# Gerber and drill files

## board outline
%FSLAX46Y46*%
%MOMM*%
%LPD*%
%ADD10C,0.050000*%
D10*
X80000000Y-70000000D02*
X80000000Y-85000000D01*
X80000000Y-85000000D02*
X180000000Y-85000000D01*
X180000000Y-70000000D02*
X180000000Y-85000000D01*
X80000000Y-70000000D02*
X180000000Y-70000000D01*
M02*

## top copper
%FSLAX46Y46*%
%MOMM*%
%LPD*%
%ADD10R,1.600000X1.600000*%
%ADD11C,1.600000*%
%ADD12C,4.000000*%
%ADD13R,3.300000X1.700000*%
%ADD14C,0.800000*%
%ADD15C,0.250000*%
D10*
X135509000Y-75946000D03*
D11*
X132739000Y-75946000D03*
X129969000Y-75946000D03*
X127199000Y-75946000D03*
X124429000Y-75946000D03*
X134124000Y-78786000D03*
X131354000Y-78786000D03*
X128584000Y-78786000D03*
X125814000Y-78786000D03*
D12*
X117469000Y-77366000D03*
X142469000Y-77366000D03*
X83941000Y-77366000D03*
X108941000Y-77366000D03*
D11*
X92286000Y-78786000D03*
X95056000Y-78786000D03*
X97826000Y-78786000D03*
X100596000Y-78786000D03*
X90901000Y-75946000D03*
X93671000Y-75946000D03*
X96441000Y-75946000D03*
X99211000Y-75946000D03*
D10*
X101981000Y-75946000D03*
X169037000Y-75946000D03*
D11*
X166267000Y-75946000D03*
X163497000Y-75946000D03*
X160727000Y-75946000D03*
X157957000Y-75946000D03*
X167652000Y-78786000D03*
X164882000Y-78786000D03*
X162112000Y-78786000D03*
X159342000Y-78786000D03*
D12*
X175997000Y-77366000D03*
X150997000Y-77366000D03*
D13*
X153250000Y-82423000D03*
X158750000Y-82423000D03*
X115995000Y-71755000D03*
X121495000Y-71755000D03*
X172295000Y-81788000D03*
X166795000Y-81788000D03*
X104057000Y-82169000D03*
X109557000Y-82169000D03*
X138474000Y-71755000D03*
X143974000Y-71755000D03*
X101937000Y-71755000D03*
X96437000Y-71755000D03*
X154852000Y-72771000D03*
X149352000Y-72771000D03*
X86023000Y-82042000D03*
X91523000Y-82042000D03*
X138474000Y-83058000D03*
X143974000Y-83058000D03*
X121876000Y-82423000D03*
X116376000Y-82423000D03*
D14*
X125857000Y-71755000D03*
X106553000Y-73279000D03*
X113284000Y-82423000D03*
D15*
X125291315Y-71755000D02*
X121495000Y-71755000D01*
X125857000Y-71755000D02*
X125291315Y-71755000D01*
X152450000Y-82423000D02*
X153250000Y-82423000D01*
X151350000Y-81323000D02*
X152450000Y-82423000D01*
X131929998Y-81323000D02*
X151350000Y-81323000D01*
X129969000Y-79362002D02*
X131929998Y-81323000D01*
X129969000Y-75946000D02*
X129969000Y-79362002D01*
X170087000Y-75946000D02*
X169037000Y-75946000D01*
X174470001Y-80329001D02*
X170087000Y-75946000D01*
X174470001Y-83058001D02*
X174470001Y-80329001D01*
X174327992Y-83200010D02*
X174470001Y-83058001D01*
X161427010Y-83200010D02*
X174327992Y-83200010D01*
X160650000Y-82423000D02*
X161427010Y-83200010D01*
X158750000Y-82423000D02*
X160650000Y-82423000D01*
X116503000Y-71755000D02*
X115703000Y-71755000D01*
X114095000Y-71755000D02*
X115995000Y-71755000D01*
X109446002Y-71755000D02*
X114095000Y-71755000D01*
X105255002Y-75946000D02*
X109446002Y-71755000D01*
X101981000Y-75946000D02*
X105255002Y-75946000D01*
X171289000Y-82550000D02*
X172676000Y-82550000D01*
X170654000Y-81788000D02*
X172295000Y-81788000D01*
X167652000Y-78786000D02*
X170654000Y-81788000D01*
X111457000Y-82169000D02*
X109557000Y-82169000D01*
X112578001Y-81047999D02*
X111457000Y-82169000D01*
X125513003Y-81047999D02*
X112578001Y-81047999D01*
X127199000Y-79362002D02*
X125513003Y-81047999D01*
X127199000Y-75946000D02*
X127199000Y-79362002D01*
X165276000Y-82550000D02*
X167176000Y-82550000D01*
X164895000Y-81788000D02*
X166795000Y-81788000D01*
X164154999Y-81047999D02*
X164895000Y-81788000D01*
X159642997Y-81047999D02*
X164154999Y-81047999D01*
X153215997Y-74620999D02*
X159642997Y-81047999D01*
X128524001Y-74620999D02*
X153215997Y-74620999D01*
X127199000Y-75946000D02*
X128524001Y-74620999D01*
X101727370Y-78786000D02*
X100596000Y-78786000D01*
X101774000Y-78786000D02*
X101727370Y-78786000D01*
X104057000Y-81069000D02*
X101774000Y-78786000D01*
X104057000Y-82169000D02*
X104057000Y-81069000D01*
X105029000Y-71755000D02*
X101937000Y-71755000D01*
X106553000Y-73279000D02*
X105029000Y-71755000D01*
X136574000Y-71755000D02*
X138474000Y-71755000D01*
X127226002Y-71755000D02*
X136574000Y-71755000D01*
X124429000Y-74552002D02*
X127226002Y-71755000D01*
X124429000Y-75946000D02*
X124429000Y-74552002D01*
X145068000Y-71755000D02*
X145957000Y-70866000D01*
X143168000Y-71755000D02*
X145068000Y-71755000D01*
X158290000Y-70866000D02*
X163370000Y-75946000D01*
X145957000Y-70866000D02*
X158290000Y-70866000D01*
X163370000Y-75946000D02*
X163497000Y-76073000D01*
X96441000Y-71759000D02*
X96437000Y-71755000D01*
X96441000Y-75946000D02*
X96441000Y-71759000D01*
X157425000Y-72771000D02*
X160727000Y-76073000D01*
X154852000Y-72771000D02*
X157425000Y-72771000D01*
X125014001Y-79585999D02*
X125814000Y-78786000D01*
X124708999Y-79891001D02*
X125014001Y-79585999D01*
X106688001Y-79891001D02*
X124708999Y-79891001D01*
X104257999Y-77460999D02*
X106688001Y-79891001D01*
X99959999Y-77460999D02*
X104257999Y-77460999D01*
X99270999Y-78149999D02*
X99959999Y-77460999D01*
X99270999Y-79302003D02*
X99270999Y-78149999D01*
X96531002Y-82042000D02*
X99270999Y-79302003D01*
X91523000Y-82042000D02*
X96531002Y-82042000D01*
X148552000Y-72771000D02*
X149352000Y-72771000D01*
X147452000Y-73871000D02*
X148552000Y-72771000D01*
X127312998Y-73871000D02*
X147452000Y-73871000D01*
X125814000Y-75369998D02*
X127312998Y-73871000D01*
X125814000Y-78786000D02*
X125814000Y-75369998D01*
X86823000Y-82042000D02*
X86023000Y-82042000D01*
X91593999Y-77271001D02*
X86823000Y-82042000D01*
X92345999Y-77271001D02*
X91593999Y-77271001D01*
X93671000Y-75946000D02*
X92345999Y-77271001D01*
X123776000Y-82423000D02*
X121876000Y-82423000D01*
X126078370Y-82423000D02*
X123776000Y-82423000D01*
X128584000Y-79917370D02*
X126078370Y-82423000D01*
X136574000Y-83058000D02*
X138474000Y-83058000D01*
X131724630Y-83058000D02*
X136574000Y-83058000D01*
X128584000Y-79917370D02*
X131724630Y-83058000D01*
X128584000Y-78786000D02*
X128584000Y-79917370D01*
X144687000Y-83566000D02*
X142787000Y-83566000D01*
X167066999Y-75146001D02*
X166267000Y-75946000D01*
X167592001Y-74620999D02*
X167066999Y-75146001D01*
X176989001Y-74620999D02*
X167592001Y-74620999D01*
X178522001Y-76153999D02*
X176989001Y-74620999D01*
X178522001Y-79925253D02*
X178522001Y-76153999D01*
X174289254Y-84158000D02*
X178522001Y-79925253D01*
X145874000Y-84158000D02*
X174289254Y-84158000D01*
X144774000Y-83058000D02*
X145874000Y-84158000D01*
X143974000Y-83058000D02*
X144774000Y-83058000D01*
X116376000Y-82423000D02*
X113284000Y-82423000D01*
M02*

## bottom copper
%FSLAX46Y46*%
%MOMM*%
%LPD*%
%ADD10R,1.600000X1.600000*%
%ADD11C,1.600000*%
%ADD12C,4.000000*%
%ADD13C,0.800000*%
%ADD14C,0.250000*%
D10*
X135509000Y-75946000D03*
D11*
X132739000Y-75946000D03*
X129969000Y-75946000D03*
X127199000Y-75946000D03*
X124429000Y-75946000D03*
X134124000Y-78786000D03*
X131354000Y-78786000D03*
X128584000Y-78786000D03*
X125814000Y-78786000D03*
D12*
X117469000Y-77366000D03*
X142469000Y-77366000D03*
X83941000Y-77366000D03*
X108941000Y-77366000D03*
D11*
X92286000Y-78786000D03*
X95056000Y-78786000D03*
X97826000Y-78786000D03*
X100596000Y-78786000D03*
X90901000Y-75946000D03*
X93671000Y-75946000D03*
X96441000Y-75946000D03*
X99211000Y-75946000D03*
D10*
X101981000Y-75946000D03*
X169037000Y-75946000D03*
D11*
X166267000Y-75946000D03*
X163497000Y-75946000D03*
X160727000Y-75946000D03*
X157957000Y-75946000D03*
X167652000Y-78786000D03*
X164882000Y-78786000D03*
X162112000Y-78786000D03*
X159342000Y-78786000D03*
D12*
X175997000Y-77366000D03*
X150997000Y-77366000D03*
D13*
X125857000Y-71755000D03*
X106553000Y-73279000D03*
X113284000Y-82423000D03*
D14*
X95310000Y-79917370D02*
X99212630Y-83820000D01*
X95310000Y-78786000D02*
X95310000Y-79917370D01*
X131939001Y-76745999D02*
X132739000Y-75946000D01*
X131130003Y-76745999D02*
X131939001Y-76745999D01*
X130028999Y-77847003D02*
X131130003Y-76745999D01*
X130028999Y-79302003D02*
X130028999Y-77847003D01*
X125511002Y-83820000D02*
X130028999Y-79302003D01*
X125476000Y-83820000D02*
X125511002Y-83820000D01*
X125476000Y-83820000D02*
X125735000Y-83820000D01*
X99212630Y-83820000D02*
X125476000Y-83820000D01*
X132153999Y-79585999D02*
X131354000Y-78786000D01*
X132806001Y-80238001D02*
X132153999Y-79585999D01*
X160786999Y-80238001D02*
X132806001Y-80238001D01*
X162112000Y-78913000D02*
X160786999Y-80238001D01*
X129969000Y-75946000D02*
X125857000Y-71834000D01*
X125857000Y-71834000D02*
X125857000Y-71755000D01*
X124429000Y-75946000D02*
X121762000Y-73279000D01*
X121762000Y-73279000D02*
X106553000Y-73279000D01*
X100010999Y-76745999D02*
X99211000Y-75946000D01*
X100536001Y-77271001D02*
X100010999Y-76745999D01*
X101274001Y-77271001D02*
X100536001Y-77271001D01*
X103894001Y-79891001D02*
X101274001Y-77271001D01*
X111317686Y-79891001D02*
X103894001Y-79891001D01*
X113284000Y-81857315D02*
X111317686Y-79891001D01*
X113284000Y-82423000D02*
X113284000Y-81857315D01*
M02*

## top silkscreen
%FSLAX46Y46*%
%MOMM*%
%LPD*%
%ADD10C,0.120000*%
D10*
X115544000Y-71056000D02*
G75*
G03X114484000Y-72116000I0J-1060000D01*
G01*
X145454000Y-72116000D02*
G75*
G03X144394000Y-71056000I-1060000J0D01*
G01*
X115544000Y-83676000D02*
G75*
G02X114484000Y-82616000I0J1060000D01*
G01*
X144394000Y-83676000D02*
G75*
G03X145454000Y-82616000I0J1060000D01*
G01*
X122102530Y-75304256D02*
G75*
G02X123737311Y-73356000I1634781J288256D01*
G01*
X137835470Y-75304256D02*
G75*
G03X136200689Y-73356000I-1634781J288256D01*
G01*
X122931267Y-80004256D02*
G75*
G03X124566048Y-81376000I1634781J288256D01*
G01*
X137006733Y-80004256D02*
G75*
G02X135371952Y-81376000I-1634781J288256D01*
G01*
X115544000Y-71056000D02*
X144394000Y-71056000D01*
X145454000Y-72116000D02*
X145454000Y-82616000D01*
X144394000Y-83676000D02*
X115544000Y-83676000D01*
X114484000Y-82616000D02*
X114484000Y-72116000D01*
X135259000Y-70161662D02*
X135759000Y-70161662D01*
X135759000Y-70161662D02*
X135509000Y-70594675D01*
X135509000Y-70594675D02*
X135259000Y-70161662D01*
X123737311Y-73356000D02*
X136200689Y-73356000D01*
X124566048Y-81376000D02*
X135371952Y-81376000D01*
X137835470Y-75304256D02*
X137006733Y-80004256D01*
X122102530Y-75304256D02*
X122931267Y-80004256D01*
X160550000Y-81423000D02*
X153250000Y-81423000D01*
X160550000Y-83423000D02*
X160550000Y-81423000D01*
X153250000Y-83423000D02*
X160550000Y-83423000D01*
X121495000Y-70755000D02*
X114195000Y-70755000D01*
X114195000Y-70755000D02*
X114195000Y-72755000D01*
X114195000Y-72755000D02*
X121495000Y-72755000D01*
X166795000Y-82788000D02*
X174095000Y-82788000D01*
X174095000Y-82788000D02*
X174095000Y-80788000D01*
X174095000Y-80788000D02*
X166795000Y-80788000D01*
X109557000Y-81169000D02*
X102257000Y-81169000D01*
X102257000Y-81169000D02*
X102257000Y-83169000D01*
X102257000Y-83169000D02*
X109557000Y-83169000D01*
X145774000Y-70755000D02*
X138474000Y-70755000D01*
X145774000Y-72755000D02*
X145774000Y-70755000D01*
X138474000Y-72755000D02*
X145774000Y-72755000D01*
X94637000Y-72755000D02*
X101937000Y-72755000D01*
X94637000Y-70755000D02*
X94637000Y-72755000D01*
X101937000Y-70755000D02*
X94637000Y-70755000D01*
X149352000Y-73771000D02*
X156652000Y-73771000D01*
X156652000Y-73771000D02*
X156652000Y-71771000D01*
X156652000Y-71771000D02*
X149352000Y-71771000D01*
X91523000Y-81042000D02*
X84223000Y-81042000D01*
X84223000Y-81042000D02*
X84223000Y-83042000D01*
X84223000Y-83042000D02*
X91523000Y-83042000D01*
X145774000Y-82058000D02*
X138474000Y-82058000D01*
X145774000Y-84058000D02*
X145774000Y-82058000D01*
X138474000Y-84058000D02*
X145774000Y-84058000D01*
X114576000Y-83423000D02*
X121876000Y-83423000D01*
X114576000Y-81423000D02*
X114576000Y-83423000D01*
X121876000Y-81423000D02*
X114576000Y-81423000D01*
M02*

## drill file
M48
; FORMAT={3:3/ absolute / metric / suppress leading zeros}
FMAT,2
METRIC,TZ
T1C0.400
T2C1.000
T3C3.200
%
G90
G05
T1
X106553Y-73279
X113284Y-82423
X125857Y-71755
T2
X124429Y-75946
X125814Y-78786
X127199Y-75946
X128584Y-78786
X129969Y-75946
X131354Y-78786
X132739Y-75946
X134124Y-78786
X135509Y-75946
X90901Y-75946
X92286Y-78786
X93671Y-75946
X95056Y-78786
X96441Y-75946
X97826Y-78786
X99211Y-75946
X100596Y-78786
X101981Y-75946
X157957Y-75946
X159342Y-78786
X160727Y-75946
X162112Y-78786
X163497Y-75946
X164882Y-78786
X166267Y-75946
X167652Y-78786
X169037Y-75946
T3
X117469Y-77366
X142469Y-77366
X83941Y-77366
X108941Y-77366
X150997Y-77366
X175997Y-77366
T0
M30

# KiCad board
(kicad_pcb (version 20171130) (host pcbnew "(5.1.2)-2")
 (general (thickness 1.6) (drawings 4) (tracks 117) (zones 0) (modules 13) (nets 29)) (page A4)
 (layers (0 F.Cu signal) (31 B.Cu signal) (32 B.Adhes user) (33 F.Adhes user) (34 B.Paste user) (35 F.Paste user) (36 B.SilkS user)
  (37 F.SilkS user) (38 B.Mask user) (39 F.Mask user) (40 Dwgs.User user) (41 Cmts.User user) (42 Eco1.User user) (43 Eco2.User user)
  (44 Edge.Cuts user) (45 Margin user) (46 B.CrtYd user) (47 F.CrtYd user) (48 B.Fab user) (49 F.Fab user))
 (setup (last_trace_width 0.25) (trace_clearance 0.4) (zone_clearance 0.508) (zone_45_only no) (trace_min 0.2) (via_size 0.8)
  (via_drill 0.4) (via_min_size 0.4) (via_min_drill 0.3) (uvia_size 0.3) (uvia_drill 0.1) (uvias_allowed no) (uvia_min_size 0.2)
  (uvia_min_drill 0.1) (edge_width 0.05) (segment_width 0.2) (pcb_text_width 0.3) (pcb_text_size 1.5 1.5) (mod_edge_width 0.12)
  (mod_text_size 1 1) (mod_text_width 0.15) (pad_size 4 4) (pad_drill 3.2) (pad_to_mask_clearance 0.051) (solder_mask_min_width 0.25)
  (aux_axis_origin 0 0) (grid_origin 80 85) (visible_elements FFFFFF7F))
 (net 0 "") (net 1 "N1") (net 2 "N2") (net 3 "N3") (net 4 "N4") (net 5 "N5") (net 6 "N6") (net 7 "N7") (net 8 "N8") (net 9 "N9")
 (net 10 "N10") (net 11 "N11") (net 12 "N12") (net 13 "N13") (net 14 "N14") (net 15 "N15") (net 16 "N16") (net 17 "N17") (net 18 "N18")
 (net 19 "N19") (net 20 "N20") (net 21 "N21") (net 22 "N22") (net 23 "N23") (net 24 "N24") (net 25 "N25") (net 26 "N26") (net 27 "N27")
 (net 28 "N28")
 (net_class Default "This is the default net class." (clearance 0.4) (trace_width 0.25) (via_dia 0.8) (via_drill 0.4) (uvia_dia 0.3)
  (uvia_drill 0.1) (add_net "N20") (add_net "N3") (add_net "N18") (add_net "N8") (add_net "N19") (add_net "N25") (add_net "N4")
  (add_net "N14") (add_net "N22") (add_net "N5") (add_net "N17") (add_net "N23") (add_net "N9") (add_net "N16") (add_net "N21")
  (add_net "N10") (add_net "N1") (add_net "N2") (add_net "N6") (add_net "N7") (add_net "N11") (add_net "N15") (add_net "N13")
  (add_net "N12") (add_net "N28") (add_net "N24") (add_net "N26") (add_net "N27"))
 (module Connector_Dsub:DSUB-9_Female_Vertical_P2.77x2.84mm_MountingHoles (layer F.Cu) (at 135.509 75.946)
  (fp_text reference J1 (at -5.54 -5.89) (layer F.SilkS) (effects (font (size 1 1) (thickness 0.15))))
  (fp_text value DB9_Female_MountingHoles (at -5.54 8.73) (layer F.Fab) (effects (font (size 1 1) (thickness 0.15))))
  (fp_arc (start -19.965 -3.83) (end -21.025 -3.83) (angle 90) (layer F.SilkS) (width 0.12))
  (fp_arc (start 8.885 -3.83) (end 8.885 -4.89) (angle 90) (layer F.SilkS) (width 0.12))
  (fp_arc (start -19.965 6.67) (end -21.025 6.67) (angle -90) (layer F.SilkS) (width 0.12))
  (fp_arc (start 8.885 6.67) (end 9.945 6.67) (angle 90) (layer F.SilkS) (width 0.12))
  (fp_arc (start -11.771689 -0.93) (end -11.771689 -2.59) (angle -100) (layer F.SilkS) (width 0.12))
  (fp_arc (start 0.691689 -0.93) (end 0.691689 -2.59) (angle 100) (layer F.SilkS) (width 0.12))
  (fp_arc (start -10.942952 3.77) (end -10.942952 5.43) (angle 80) (layer F.SilkS) (width 0.12))
  (fp_arc (start -0.137048 3.77) (end -0.137048 5.43) (angle -80) (layer F.SilkS) (width 0.12))
  (fp_line (start -19.965 -4.89) (end 8.885 -4.89) (layer F.SilkS) (width 0.12))
  (fp_line (start 9.945 -3.83) (end 9.945 6.67) (layer F.SilkS) (width 0.12))
  (fp_line (start 8.885 7.73) (end -19.965 7.73) (layer F.SilkS) (width 0.12))
  (fp_line (start -21.025 6.67) (end -21.025 -3.83) (layer F.SilkS) (width 0.12))
  (fp_line (start -0.25 -5.784338) (end 0.25 -5.784338) (layer F.SilkS) (width 0.12))
  (fp_line (start 0.25 -5.784338) (end 0 -5.351325) (layer F.SilkS) (width 0.12))
  (fp_line (start 0 -5.351325) (end -0.25 -5.784338) (layer F.SilkS) (width 0.12))
  (fp_line (start -11.771689 -2.59) (end 0.691689 -2.59) (layer F.SilkS) (width 0.12))
  (fp_line (start -10.942952 5.43) (end -0.137048 5.43) (layer F.SilkS) (width 0.12))
  (fp_line (start 2.32647 -0.641744) (end 1.497733 4.058256) (layer F.SilkS) (width 0.12))
  (fp_line (start -13.40647 -0.641744) (end -12.577733 4.058256) (layer F.SilkS) (width 0.12))
  (pad 1 thru_hole rect (at 0 0) (size 1.6 1.6) (drill 1) (layers *.Cu *.Mask) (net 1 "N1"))
  (pad 2 thru_hole circle (at -2.77 0) (size 1.6 1.6) (drill 1) (layers *.Cu *.Mask) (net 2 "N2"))
  (pad 3 thru_hole circle (at -5.54 0) (size 1.6 1.6) (drill 1) (layers *.Cu *.Mask) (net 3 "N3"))
  (pad 4 thru_hole circle (at -8.31 0) (size 1.6 1.6) (drill 1) (layers *.Cu *.Mask) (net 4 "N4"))
  (pad 5 thru_hole circle (at -11.08 0) (size 1.6 1.6) (drill 1) (layers *.Cu *.Mask) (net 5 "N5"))
  (pad 6 thru_hole circle (at -1.385 2.84) (size 1.6 1.6) (drill 1) (layers *.Cu *.Mask) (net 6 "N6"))
  (pad 7 thru_hole circle (at -4.155 2.84) (size 1.6 1.6) (drill 1) (layers *.Cu *.Mask) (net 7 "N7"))
  (pad 8 thru_hole circle (at -6.925 2.84) (size 1.6 1.6) (drill 1) (layers *.Cu *.Mask) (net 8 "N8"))
  (pad 9 thru_hole circle (at -9.695 2.84) (size 1.6 1.6) (drill 1) (layers *.Cu *.Mask) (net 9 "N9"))
  (pad 0 thru_hole circle (at -18.04 1.42) (size 4 4) (drill 3.2) (layers *.Cu *.Mask) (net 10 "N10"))
  (pad 0 thru_hole circle (at 6.96 1.42) (size 4 4) (drill 3.2) (layers *.Cu *.Mask) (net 10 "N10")))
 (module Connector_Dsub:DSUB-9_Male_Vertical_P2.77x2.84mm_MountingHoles (layer B.Cu) (at 101.981 75.946 180)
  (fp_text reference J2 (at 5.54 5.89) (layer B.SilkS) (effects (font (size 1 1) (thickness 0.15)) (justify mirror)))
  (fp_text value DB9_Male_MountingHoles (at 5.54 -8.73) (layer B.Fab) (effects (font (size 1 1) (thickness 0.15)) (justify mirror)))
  (pad 0 thru_hole circle (at 18.04 -1.42 180) (size 4 4) (drill 3.2) (layers *.Cu *.Mask) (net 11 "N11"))
  (pad 0 thru_hole circle (at -6.96 -1.42 180) (size 4 4) (drill 3.2) (layers *.Cu *.Mask) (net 11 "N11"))
  (pad 9 thru_hole circle (at 9.695 -2.84 180) (size 1.6 1.6) (drill 1) (layers *.Cu *.Mask) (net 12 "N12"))
  (pad 8 thru_hole circle (at 6.925 -2.84 180) (size 1.6 1.6) (drill 1) (layers *.Cu *.Mask) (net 2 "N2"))
  (pad 7 thru_hole circle (at 4.155 -2.84 180) (size 1.6 1.6) (drill 1) (layers *.Cu *.Mask) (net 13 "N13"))
  (pad 6 thru_hole circle (at 1.385 -2.84 180) (size 1.6 1.6) (drill 1) (layers *.Cu *.Mask) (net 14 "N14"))
  (pad 5 thru_hole circle (at 11.08 0 180) (size 1.6 1.6) (drill 1) (layers *.Cu *.Mask) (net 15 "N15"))
  (pad 4 thru_hole circle (at 8.31 0 180) (size 1.6 1.6) (drill 1) (layers *.Cu *.Mask) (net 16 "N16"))
  (pad 3 thru_hole circle (at 5.54 0 180) (size 1.6 1.6) (drill 1) (layers *.Cu *.Mask) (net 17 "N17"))
  (pad 2 thru_hole circle (at 2.77 0 180) (size 1.6 1.6) (drill 1) (layers *.Cu *.Mask) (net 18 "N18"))
  (pad 1 thru_hole rect (at 0 0 180) (size 1.6 1.6) (drill 1) (layers *.Cu *.Mask) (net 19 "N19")))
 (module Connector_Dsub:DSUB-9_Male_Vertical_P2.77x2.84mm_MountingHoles (layer B.Cu) (at 169.037 75.946 180)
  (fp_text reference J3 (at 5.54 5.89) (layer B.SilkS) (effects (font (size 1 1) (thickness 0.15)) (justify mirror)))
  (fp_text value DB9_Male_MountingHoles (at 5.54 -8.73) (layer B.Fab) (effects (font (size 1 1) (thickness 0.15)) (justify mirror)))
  (pad 1 thru_hole rect (at 0 0 180) (size 1.6 1.6) (drill 1) (layers *.Cu *.Mask) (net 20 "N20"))
  (pad 2 thru_hole circle (at 2.77 0 180) (size 1.6 1.6) (drill 1) (layers *.Cu *.Mask) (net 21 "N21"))
  (pad 3 thru_hole circle (at 5.54 0 180) (size 1.6 1.6) (drill 1) (layers *.Cu *.Mask) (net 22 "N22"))
  (pad 4 thru_hole circle (at 8.31 0 180) (size 1.6 1.6) (drill 1) (layers *.Cu *.Mask) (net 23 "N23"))
  (pad 5 thru_hole circle (at 11.08 0 180) (size 1.6 1.6) (drill 1) (layers *.Cu *.Mask) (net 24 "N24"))
  (pad 6 thru_hole circle (at 1.385 -2.84 180) (size 1.6 1.6) (drill 1) (layers *.Cu *.Mask) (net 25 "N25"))
  (pad 7 thru_hole circle (at 4.155 -2.84 180) (size 1.6 1.6) (drill 1) (layers *.Cu *.Mask) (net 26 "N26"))
  (pad 8 thru_hole circle (at 6.925 -2.84 180) (size 1.6 1.6) (drill 1) (layers *.Cu *.Mask) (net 7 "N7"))
  (pad 9 thru_hole circle (at 9.695 -2.84 180) (size 1.6 1.6) (drill 1) (layers *.Cu *.Mask) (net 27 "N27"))
  (pad 0 thru_hole circle (at -6.96 -1.42 180) (size 4 4) (drill 3.2) (layers *.Cu *.Mask) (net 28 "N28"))
  (pad 0 thru_hole circle (at 18.04 -1.42 180) (size 4 4) (drill 3.2) (layers *.Cu *.Mask) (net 28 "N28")))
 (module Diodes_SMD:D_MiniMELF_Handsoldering (layer F.Cu) (at 156 82.423 180)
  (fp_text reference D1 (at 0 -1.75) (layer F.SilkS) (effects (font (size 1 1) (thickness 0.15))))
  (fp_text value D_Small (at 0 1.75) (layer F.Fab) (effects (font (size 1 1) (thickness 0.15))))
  (fp_line (start -4.55 1) (end 2.75 1) (layer F.SilkS) (width 0.12))
  (fp_line (start -4.55 -1) (end -4.55 1) (layer F.SilkS) (width 0.12))
  (fp_line (start 2.75 -1) (end -4.55 -1) (layer F.SilkS) (width 0.12))
  (pad 2 smd rect (at 2.75 0 180) (size 3.3 1.7) (layers F.Cu F.Paste F.Mask) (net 3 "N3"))
  (pad 1 smd rect (at -2.75 0 180) (size 3.3 1.7) (layers F.Cu F.Paste F.Mask) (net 20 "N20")))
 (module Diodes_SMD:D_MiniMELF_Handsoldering (layer F.Cu) (at 118.745 71.755)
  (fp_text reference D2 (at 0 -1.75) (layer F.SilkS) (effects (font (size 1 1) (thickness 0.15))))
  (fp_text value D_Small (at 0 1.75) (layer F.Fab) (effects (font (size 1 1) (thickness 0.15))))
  (fp_line (start 2.75 -1) (end -4.55 -1) (layer F.SilkS) (width 0.12))
  (fp_line (start -4.55 -1) (end -4.55 1) (layer F.SilkS) (width 0.12))
  (fp_line (start -4.55 1) (end 2.75 1) (layer F.SilkS) (width 0.12))
  (pad 1 smd rect (at -2.75 0) (size 3.3 1.7) (layers F.Cu F.Paste F.Mask) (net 19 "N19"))
  (pad 2 smd rect (at 2.75 0) (size 3.3 1.7) (layers F.Cu F.Paste F.Mask) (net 3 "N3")))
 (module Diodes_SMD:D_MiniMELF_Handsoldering (layer F.Cu) (at 169.545 81.788 180)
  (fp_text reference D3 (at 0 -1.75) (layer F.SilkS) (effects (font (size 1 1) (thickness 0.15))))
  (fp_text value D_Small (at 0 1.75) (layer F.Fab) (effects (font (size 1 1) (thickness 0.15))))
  (fp_line (start 2.75 -1) (end -4.55 -1) (layer F.SilkS) (width 0.12))
  (fp_line (start -4.55 -1) (end -4.55 1) (layer F.SilkS) (width 0.12))
  (fp_line (start -4.55 1) (end 2.75 1) (layer F.SilkS) (width 0.12))
  (pad 1 smd rect (at -2.75 0 180) (size 3.3 1.7) (layers F.Cu F.Paste F.Mask) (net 25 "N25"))
  (pad 2 smd rect (at 2.75 0 180) (size 3.3 1.7) (layers F.Cu F.Paste F.Mask) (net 4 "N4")))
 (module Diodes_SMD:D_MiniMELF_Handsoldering (layer F.Cu) (at 106.807 82.169)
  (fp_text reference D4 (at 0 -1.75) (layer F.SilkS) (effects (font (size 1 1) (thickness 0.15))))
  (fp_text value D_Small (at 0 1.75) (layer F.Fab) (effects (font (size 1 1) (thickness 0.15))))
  (fp_line (start 2.75 -1) (end -4.55 -1) (layer F.SilkS) (width 0.12))
  (fp_line (start -4.55 -1) (end -4.55 1) (layer F.SilkS) (width 0.12))
  (fp_line (start -4.55 1) (end 2.75 1) (layer F.SilkS) (width 0.12))
  (pad 1 smd rect (at -2.75 0) (size 3.3 1.7) (layers F.Cu F.Paste F.Mask) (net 14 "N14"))
  (pad 2 smd rect (at 2.75 0) (size 3.3 1.7) (layers F.Cu F.Paste F.Mask) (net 4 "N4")))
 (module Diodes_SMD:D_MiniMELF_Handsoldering (layer F.Cu) (at 141.224 71.755 180)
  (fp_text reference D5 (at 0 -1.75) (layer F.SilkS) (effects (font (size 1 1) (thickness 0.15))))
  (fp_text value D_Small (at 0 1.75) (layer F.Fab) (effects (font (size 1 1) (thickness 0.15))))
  (fp_line (start -4.55 1) (end 2.75 1) (layer F.SilkS) (width 0.12))
  (fp_line (start -4.55 -1) (end -4.55 1) (layer F.SilkS) (width 0.12))
  (fp_line (start 2.75 -1) (end -4.55 -1) (layer F.SilkS) (width 0.12))
  (pad 2 smd rect (at 2.75 0 180) (size 3.3 1.7) (layers F.Cu F.Paste F.Mask) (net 5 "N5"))
  (pad 1 smd rect (at -2.75 0 180) (size 3.3 1.7) (layers F.Cu F.Paste F.Mask) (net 22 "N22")))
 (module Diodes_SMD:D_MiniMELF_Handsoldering (layer F.Cu) (at 99.187 71.755)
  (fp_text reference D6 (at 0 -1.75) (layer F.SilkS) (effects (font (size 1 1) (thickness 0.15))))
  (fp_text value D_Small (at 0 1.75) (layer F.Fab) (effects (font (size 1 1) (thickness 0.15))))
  (fp_line (start -4.55 1) (end 2.75 1) (layer F.SilkS) (width 0.12))
  (fp_line (start -4.55 -1) (end -4.55 1) (layer F.SilkS) (width 0.12))
  (fp_line (start 2.75 -1) (end -4.55 -1) (layer F.SilkS) (width 0.12))
  (pad 2 smd rect (at 2.75 0) (size 3.3 1.7) (layers F.Cu F.Paste F.Mask) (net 5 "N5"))
  (pad 1 smd rect (at -2.75 0) (size 3.3 1.7) (layers F.Cu F.Paste F.Mask) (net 17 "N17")))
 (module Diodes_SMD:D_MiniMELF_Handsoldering (layer F.Cu) (at 152.102 72.771 180)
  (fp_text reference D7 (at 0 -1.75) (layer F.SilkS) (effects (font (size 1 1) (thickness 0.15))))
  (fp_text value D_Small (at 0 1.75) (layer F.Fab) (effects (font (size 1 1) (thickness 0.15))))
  (fp_line (start 2.75 -1) (end -4.55 -1) (layer F.SilkS) (width 0.12))
  (fp_line (start -4.55 -1) (end -4.55 1) (layer F.SilkS) (width 0.12))
  (fp_line (start -4.55 1) (end 2.75 1) (layer F.SilkS) (width 0.12))
  (pad 1 smd rect (at -2.75 0 180) (size 3.3 1.7) (layers F.Cu F.Paste F.Mask) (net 23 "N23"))
  (pad 2 smd rect (at 2.75 0 180) (size 3.3 1.7) (layers F.Cu F.Paste F.Mask) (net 9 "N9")))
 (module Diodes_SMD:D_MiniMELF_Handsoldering (layer F.Cu) (at 88.773 82.042)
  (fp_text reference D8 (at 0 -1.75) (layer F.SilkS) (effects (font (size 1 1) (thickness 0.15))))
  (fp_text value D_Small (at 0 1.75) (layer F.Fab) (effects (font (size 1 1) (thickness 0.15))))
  (fp_line (start 2.75 -1) (end -4.55 -1) (layer F.SilkS) (width 0.12))
  (fp_line (start -4.55 -1) (end -4.55 1) (layer F.SilkS) (width 0.12))
  (fp_line (start -4.55 1) (end 2.75 1) (layer F.SilkS) (width 0.12))
  (pad 1 smd rect (at -2.75 0) (size 3.3 1.7) (layers F.Cu F.Paste F.Mask) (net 16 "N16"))
  (pad 2 smd rect (at 2.75 0) (size 3.3 1.7) (layers F.Cu F.Paste F.Mask) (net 9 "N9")))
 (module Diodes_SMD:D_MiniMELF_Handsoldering (layer F.Cu) (at 141.224 83.058 180)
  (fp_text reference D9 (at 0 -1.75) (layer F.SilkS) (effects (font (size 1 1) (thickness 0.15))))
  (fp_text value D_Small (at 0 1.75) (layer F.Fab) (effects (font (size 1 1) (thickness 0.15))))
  (fp_line (start -4.55 1) (end 2.75 1) (layer F.SilkS) (width 0.12))
  (fp_line (start -4.55 -1) (end -4.55 1) (layer F.SilkS) (width 0.12))
  (fp_line (start 2.75 -1) (end -4.55 -1) (layer F.SilkS) (width 0.12))
  (pad 2 smd rect (at 2.75 0 180) (size 3.3 1.7) (layers F.Cu F.Paste F.Mask) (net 8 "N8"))
  (pad 1 smd rect (at -2.75 0 180) (size 3.3 1.7) (layers F.Cu F.Paste F.Mask) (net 21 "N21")))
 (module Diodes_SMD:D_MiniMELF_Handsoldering (layer F.Cu) (at 119.126 82.423)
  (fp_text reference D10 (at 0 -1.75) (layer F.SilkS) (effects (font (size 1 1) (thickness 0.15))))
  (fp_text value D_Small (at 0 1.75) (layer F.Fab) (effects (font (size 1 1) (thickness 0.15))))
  (fp_line (start -4.55 1) (end 2.75 1) (layer F.SilkS) (width 0.12))
  (fp_line (start -4.55 -1) (end -4.55 1) (layer F.SilkS) (width 0.12))
  (fp_line (start 2.75 -1) (end -4.55 -1) (layer F.SilkS) (width 0.12))
  (pad 2 smd rect (at 2.75 0) (size 3.3 1.7) (layers F.Cu F.Paste F.Mask) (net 8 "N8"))
  (pad 1 smd rect (at -2.75 0) (size 3.3 1.7) (layers F.Cu F.Paste F.Mask) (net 18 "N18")))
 (gr_line (start 80 70) (end 80 85) (layer Edge.Cuts) (width 0.05))
 (gr_line (start 80 85) (end 180 85) (layer Edge.Cuts) (width 0.05))
 (gr_line (start 180 70) (end 180 85) (layer Edge.Cuts) (width 0.05))
 (gr_line (start 80 70) (end 180 70) (layer Edge.Cuts) (width 0.05))
 (segment (start 95.31 79.91737) (end 99.21263 83.82) (width 0.25) (layer B.Cu) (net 2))
 (segment (start 95.31 78.786) (end 95.31 79.91737) (width 0.25) (layer B.Cu) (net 2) (status 10))
 (segment (start 131.939001 76.745999) (end 132.739 75.946) (width 0.25) (layer B.Cu) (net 2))
 (segment (start 131.130003 76.745999) (end 131.939001 76.745999) (width 0.25) (layer B.Cu) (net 2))
 (segment (start 130.028999 77.847003) (end 131.130003 76.745999) (width 0.25) (layer B.Cu) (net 2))
 (segment (start 130.028999 79.302003) (end 130.028999 77.847003) (width 0.25) (layer B.Cu) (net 2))
 (segment (start 125.511002 83.82) (end 130.028999 79.302003) (width 0.25) (layer B.Cu) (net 2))
 (segment (start 125.476 83.82) (end 125.511002 83.82) (width 0.25) (layer B.Cu) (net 2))
 (segment (start 125.476 83.82) (end 125.735 83.82) (width 0.25) (layer B.Cu) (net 2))
 (segment (start 99.21263 83.82) (end 125.476 83.82) (width 0.25) (layer B.Cu) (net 2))
 (segment (start 132.153999 79.585999) (end 131.354 78.786) (width 0.25) (layer B.Cu) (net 7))
 (segment (start 132.806001 80.238001) (end 132.153999 79.585999) (width 0.25) (layer B.Cu) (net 7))
 (segment (start 160.786999 80.238001) (end 132.806001 80.238001) (width 0.25) (layer B.Cu) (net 7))
 (segment (start 162.112 78.913) (end 160.786999 80.238001) (width 0.25) (layer B.Cu) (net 7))
 (via (at 125.857 71.755) (size 0.8) (drill 0.4) (layers F.Cu B.Cu) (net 3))
 (segment (start 129.969 75.946) (end 125.857 71.834) (width 0.25) (layer B.Cu) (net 3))
 (segment (start 125.857 71.834) (end 125.857 71.755) (width 0.25) (layer B.Cu) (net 3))
 (segment (start 125.291315 71.755) (end 121.495 71.755) (width 0.25) (layer F.Cu) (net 3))
 (segment (start 125.857 71.755) (end 125.291315 71.755) (width 0.25) (layer F.Cu) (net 3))
 (segment (start 152.45 82.423) (end 153.25 82.423) (width 0.25) (layer F.Cu) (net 3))
 (segment (start 151.35 81.323) (end 152.45 82.423) (width 0.25) (layer F.Cu) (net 3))
 (segment (start 131.929998 81.323) (end 151.35 81.323) (width 0.25) (layer F.Cu) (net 3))
 (segment (start 129.969 79.362002) (end 131.929998 81.323) (width 0.25) (layer F.Cu) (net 3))
 (segment (start 129.969 75.946) (end 129.969 79.362002) (width 0.25) (layer F.Cu) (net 3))
 (segment (start 170.087 75.946) (end 169.037 75.946) (width 0.25) (layer F.Cu) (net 20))
 (segment (start 174.470001 80.329001) (end 170.087 75.946) (width 0.25) (layer F.Cu) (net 20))
 (segment (start 174.470001 83.058001) (end 174.470001 80.329001) (width 0.25) (layer F.Cu) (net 20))
 (segment (start 174.327992 83.20001) (end 174.470001 83.058001) (width 0.25) (layer F.Cu) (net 20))
 (segment (start 161.42701 83.20001) (end 174.327992 83.20001) (width 0.25) (layer F.Cu) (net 20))
 (segment (start 160.65 82.423) (end 161.42701 83.20001) (width 0.25) (layer F.Cu) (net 20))
 (segment (start 158.75 82.423) (end 160.65 82.423) (width 0.25) (layer F.Cu) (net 20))
 (segment (start 116.503 71.755) (end 115.703 71.755) (width 0.25) (layer F.Cu) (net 19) (status 30))
 (segment (start 114.095 71.755) (end 115.995 71.755) (width 0.25) (layer F.Cu) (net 19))
 (segment (start 109.446002 71.755) (end 114.095 71.755) (width 0.25) (layer F.Cu) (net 19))
 (segment (start 105.255002 75.946) (end 109.446002 71.755) (width 0.25) (layer F.Cu) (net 19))
 (segment (start 101.981 75.946) (end 105.255002 75.946) (width 0.25) (layer F.Cu) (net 19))
 (segment (start 171.289 82.55) (end 172.676 82.55) (width 0.25) (layer F.Cu) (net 25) (status 30))
 (segment (start 170.654 81.788) (end 172.295 81.788) (width 0.25) (layer F.Cu) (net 25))
 (segment (start 167.652 78.786) (end 170.654 81.788) (width 0.25) (layer F.Cu) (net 25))
 (segment (start 111.457 82.169) (end 109.557 82.169) (width 0.25) (layer F.Cu) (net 4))
 (segment (start 112.578001 81.047999) (end 111.457 82.169) (width 0.25) (layer F.Cu) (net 4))
 (segment (start 125.513003 81.047999) (end 112.578001 81.047999) (width 0.25) (layer F.Cu) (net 4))
 (segment (start 127.199 79.362002) (end 125.513003 81.047999) (width 0.25) (layer F.Cu) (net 4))
 (segment (start 127.199 75.946) (end 127.199 79.362002) (width 0.25) (layer F.Cu) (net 4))
 (segment (start 165.276 82.55) (end 167.176 82.55) (width 0.25) (layer F.Cu) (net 4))
 (segment (start 164.895 81.788) (end 166.795 81.788) (width 0.25) (layer F.Cu) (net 4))
 (segment (start 164.154999 81.047999) (end 164.895 81.788) (width 0.25) (layer F.Cu) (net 4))
 (segment (start 159.642997 81.047999) (end 164.154999 81.047999) (width 0.25) (layer F.Cu) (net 4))
 (segment (start 153.215997 74.620999) (end 159.642997 81.047999) (width 0.25) (layer F.Cu) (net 4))
 (segment (start 128.524001 74.620999) (end 153.215997 74.620999) (width 0.25) (layer F.Cu) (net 4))
 (segment (start 127.199 75.946) (end 128.524001 74.620999) (width 0.25) (layer F.Cu) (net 4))
 (segment (start 101.72737 78.786) (end 100.596 78.786) (width 0.25) (layer F.Cu) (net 14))
 (segment (start 101.774 78.786) (end 101.72737 78.786) (width 0.25) (layer F.Cu) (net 14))
 (segment (start 104.057 81.069) (end 101.774 78.786) (width 0.25) (layer F.Cu) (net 14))
 (segment (start 104.057 82.169) (end 104.057 81.069) (width 0.25) (layer F.Cu) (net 14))
 (via (at 106.553 73.279) (size 0.8) (drill 0.4) (layers F.Cu B.Cu) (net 5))
 (segment (start 124.429 75.946) (end 121.762 73.279) (width 0.25) (layer B.Cu) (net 5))
 (segment (start 121.762 73.279) (end 106.553 73.279) (width 0.25) (layer B.Cu) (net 5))
 (segment (start 105.029 71.755) (end 101.937 71.755) (width 0.25) (layer F.Cu) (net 5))
 (segment (start 106.553 73.279) (end 105.029 71.755) (width 0.25) (layer F.Cu) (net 5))
 (segment (start 136.574 71.755) (end 138.474 71.755) (width 0.25) (layer F.Cu) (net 5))
 (segment (start 127.226002 71.755) (end 136.574 71.755) (width 0.25) (layer F.Cu) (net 5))
 (segment (start 124.429 74.552002) (end 127.226002 71.755) (width 0.25) (layer F.Cu) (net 5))
 (segment (start 124.429 75.946) (end 124.429 74.552002) (width 0.25) (layer F.Cu) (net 5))
 (segment (start 145.068 71.755) (end 145.957 70.866) (width 0.25) (layer F.Cu) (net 22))
 (segment (start 143.168 71.755) (end 145.068 71.755) (width 0.25) (layer F.Cu) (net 22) (status 10))
 (segment (start 158.29 70.866) (end 163.37 75.946) (width 0.25) (layer F.Cu) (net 22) (status 20))
 (segment (start 145.957 70.866) (end 158.29 70.866) (width 0.25) (layer F.Cu) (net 22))
 (segment (start 163.37 75.946) (end 163.497 76.073) (width 0.25) (layer F.Cu) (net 22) (status 30))
 (segment (start 96.441 71.759) (end 96.437 71.755) (width 0.25) (layer F.Cu) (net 17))
 (segment (start 96.441 75.946) (end 96.441 71.759) (width 0.25) (layer F.Cu) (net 17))
 (segment (start 157.425 72.771) (end 160.727 76.073) (width 0.25) (layer F.Cu) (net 23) (status 20))
 (segment (start 154.852 72.771) (end 157.425 72.771) (width 0.25) (layer F.Cu) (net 23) (status 10))
 (segment (start 125.014001 79.585999) (end 125.814 78.786) (width 0.25) (layer F.Cu) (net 9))
 (segment (start 124.708999 79.891001) (end 125.014001 79.585999) (width 0.25) (layer F.Cu) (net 9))
 (segment (start 106.688001 79.891001) (end 124.708999 79.891001) (width 0.25) (layer F.Cu) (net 9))
 (segment (start 104.257999 77.460999) (end 106.688001 79.891001) (width 0.25) (layer F.Cu) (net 9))
 (segment (start 99.959999 77.460999) (end 104.257999 77.460999) (width 0.25) (layer F.Cu) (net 9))
 (segment (start 99.270999 78.149999) (end 99.959999 77.460999) (width 0.25) (layer F.Cu) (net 9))
 (segment (start 99.270999 79.302003) (end 99.270999 78.149999) (width 0.25) (layer F.Cu) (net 9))
 (segment (start 96.531002 82.042) (end 99.270999 79.302003) (width 0.25) (layer F.Cu) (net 9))
 (segment (start 91.523 82.042) (end 96.531002 82.042) (width 0.25) (layer F.Cu) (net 9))
 (segment (start 148.552 72.771) (end 149.352 72.771) (width 0.25) (layer F.Cu) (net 9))
 (segment (start 147.452 73.871) (end 148.552 72.771) (width 0.25) (layer F.Cu) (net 9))
 (segment (start 127.312998 73.871) (end 147.452 73.871) (width 0.25) (layer F.Cu) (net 9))
 (segment (start 125.814 75.369998) (end 127.312998 73.871) (width 0.25) (layer F.Cu) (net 9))
 (segment (start 125.814 78.786) (end 125.814 75.369998) (width 0.25) (layer F.Cu) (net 9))
 (segment (start 86.823 82.042) (end 86.023 82.042) (width 0.25) (layer F.Cu) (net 16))
 (segment (start 91.593999 77.271001) (end 86.823 82.042) (width 0.25) (layer F.Cu) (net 16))
 (segment (start 92.345999 77.271001) (end 91.593999 77.271001) (width 0.25) (layer F.Cu) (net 16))
 (segment (start 93.671 75.946) (end 92.345999 77.271001) (width 0.25) (layer F.Cu) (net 16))
 (segment (start 123.776 82.423) (end 121.876 82.423) (width 0.25) (layer F.Cu) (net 8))
 (segment (start 126.07837 82.423) (end 123.776 82.423) (width 0.25) (layer F.Cu) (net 8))
 (segment (start 128.584 79.91737) (end 126.07837 82.423) (width 0.25) (layer F.Cu) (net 8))
 (segment (start 136.574 83.058) (end 138.474 83.058) (width 0.25) (layer F.Cu) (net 8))
 (segment (start 131.72463 83.058) (end 136.574 83.058) (width 0.25) (layer F.Cu) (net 8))
 (segment (start 128.584 79.91737) (end 131.72463 83.058) (width 0.25) (layer F.Cu) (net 8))
 (segment (start 128.584 78.786) (end 128.584 79.91737) (width 0.25) (layer F.Cu) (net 8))
 (segment (start 144.687 83.566) (end 142.787 83.566) (width 0.25) (layer F.Cu) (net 21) (status 20))
 (segment (start 167.066999 75.146001) (end 166.267 75.946) (width 0.25) (layer F.Cu) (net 21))
 (segment (start 167.592001 74.620999) (end 167.066999 75.146001) (width 0.25) (layer F.Cu) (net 21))
 (segment (start 176.989001 74.620999) (end 167.592001 74.620999) (width 0.25) (layer F.Cu) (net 21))
 (segment (start 178.522001 76.153999) (end 176.989001 74.620999) (width 0.25) (layer F.Cu) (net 21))
 (segment (start 178.522001 79.925253) (end 178.522001 76.153999) (width 0.25) (layer F.Cu) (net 21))
 (segment (start 174.289254 84.158) (end 178.522001 79.925253) (width 0.25) (layer F.Cu) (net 21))
 (segment (start 145.874 84.158) (end 174.289254 84.158) (width 0.25) (layer F.Cu) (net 21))
 (segment (start 144.774 83.058) (end 145.874 84.158) (width 0.25) (layer F.Cu) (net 21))
 (segment (start 143.974 83.058) (end 144.774 83.058) (width 0.25) (layer F.Cu) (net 21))
 (via (at 113.284 82.423) (size 0.8) (drill 0.4) (layers F.Cu B.Cu) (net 18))
 (segment (start 116.376 82.423) (end 113.284 82.423) (width 0.25) (layer F.Cu) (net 18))
 (segment (start 100.010999 76.745999) (end 99.211 75.946) (width 0.25) (layer B.Cu) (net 18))
 (segment (start 100.536001 77.271001) (end 100.010999 76.745999) (width 0.25) (layer B.Cu) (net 18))
 (segment (start 101.274001 77.271001) (end 100.536001 77.271001) (width 0.25) (layer B.Cu) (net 18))
 (segment (start 103.894001 79.891001) (end 101.274001 77.271001) (width 0.25) (layer B.Cu) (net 18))
 (segment (start 111.317686 79.891001) (end 103.894001 79.891001) (width 0.25) (layer B.Cu) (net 18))
 (segment (start 113.284 81.857315) (end 111.317686 79.891001) (width 0.25) (layer B.Cu) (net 18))
 (segment (start 113.284 82.423) (end 113.284 81.857315) (width 0.25) (layer B.Cu) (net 18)))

